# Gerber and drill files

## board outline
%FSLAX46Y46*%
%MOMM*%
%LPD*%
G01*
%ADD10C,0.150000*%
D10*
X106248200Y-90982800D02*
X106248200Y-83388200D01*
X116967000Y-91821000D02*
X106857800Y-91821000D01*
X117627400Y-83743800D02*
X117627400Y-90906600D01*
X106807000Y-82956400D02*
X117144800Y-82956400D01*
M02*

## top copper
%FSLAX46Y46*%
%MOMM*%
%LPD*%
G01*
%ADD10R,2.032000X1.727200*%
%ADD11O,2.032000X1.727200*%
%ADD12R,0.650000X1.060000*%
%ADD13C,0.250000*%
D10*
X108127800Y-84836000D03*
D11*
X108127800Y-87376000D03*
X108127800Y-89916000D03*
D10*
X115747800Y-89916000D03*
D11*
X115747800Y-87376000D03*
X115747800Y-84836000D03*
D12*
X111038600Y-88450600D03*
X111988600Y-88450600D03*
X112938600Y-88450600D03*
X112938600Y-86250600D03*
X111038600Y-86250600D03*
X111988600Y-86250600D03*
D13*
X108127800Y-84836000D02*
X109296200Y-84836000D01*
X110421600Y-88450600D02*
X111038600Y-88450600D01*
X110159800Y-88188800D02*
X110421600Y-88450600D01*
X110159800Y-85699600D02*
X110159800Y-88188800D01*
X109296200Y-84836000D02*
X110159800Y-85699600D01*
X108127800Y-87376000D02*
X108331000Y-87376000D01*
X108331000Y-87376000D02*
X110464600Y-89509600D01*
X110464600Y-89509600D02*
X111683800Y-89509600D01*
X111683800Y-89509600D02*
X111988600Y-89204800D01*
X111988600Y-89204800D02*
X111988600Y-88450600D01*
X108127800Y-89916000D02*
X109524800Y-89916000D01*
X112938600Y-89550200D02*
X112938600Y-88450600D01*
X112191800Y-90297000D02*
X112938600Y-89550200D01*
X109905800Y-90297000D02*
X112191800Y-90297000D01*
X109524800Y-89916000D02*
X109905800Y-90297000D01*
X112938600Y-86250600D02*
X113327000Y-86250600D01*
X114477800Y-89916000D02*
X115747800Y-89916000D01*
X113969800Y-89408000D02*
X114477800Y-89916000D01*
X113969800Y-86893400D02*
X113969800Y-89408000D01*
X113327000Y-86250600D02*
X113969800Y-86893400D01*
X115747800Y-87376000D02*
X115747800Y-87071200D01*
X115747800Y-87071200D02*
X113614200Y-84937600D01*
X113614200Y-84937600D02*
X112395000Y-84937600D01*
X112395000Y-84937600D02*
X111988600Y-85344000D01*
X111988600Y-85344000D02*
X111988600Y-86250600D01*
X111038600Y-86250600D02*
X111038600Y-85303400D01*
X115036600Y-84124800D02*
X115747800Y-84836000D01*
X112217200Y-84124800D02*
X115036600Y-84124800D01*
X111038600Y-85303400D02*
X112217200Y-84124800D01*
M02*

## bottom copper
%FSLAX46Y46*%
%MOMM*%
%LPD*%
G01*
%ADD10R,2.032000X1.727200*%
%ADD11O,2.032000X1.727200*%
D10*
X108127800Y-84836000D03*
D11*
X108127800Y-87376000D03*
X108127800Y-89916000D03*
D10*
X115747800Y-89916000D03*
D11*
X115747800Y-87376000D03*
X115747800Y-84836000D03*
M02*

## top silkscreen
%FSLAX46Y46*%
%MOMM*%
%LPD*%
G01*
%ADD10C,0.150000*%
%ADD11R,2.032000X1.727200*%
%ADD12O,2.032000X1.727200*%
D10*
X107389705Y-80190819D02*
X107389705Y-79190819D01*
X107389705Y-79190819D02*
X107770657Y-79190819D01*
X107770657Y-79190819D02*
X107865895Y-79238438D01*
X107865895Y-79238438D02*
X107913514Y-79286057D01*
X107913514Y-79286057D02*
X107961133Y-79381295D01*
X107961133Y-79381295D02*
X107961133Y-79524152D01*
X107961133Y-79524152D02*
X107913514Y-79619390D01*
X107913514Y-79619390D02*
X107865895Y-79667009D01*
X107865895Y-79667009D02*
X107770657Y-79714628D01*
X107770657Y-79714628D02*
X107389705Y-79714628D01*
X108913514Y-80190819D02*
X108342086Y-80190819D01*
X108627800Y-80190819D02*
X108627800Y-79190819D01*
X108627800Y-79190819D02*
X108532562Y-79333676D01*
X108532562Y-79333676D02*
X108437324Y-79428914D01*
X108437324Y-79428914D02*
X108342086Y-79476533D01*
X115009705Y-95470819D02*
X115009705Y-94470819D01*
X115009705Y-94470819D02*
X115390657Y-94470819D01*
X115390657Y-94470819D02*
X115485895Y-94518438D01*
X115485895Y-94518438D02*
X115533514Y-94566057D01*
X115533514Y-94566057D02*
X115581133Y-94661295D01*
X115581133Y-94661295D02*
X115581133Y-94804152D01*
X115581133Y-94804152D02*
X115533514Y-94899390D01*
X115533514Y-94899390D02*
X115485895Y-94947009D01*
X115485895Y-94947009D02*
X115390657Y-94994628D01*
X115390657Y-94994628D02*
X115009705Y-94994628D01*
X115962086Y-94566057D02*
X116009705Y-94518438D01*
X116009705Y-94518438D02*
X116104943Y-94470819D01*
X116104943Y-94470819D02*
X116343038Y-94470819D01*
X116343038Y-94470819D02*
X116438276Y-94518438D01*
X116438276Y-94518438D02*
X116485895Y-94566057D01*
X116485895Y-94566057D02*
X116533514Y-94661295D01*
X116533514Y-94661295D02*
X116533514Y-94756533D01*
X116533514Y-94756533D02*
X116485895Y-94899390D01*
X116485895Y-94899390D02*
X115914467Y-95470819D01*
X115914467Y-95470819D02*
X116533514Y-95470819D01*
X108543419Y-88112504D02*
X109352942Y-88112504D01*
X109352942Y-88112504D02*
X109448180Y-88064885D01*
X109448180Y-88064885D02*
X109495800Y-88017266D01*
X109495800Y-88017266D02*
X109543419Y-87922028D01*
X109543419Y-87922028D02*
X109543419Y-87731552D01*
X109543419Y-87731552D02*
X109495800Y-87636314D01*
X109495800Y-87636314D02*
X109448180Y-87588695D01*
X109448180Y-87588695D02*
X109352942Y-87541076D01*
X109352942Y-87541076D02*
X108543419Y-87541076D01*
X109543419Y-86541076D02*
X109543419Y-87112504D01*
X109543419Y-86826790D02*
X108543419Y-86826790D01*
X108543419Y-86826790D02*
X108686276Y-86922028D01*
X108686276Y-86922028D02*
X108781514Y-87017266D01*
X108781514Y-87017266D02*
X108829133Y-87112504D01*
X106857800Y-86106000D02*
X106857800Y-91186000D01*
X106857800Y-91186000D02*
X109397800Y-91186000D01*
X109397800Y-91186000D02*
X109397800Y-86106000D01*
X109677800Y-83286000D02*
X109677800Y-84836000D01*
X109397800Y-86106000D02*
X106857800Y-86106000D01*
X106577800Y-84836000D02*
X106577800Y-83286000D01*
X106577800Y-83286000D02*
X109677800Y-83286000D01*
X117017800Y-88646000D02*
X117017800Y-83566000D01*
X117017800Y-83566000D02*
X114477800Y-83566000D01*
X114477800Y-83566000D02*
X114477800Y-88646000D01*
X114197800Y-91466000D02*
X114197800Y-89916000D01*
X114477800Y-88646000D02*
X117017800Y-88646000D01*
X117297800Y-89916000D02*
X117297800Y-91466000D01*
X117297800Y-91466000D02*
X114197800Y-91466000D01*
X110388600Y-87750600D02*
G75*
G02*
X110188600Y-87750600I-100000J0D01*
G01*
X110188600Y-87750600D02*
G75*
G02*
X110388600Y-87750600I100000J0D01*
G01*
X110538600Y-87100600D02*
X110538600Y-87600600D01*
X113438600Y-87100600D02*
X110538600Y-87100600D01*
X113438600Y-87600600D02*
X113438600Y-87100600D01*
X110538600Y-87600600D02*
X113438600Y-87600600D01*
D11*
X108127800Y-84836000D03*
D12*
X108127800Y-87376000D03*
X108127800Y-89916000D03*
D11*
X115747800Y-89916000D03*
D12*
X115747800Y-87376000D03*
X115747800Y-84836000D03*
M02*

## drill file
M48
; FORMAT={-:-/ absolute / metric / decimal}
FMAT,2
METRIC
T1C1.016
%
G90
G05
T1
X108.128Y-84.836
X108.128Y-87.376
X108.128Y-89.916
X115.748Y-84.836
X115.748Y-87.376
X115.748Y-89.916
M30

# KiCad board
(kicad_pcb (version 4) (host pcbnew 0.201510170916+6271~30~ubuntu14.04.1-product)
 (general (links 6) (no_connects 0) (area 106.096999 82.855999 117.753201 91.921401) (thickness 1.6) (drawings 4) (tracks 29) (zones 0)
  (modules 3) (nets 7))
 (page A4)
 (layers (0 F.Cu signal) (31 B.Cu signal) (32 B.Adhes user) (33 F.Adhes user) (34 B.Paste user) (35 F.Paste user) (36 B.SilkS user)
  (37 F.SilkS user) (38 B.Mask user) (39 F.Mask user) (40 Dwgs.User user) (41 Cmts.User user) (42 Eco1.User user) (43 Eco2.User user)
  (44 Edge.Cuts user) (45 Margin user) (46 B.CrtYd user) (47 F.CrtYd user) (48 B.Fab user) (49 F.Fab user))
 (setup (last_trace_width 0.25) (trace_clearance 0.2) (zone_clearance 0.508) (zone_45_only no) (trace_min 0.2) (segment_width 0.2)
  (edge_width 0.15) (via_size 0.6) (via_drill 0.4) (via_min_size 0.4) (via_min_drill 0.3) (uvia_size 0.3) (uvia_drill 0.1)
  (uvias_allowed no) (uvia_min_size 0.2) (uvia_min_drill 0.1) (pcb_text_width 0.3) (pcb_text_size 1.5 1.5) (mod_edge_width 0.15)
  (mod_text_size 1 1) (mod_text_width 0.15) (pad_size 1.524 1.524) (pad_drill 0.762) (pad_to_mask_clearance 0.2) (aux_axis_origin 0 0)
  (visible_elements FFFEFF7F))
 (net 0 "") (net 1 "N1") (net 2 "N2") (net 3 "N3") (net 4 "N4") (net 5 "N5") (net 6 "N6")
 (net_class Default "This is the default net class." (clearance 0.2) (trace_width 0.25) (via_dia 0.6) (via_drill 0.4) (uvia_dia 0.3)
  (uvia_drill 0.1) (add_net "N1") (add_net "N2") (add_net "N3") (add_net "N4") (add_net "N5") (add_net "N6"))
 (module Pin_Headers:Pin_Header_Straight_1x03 (layer F.Cu) (at 108.1278 84.836)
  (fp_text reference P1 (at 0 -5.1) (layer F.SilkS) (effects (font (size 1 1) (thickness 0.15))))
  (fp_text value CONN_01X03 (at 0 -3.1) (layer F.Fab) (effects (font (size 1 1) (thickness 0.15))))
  (fp_line (start -1.27 1.27) (end -1.27 6.35) (layer F.SilkS) (width 0.15))
  (fp_line (start -1.27 6.35) (end 1.27 6.35) (layer F.SilkS) (width 0.15))
  (fp_line (start 1.27 6.35) (end 1.27 1.27) (layer F.SilkS) (width 0.15))
  (fp_line (start 1.55 -1.55) (end 1.55 0) (layer F.SilkS) (width 0.15))
  (fp_line (start 1.27 1.27) (end -1.27 1.27) (layer F.SilkS) (width 0.15))
  (fp_line (start -1.55 0) (end -1.55 -1.55) (layer F.SilkS) (width 0.15))
  (fp_line (start -1.55 -1.55) (end 1.55 -1.55) (layer F.SilkS) (width 0.15))
  (pad 1 thru_hole rect (at 0 0) (size 2.032 1.7272) (drill 1.016) (layers *.Cu *.Mask F.SilkS) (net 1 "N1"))
  (pad 2 thru_hole oval (at 0 2.54) (size 2.032 1.7272) (drill 1.016) (layers *.Cu *.Mask F.SilkS) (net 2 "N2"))
  (pad 3 thru_hole oval (at 0 5.08) (size 2.032 1.7272) (drill 1.016) (layers *.Cu *.Mask F.SilkS) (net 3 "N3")))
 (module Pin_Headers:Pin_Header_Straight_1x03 (layer F.Cu) (at 115.7478 89.916 180)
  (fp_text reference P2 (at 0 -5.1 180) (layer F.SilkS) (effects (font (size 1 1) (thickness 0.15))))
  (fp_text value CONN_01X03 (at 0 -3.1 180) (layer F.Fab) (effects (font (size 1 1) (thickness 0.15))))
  (fp_line (start -1.27 1.27) (end -1.27 6.35) (layer F.SilkS) (width 0.15))
  (fp_line (start -1.27 6.35) (end 1.27 6.35) (layer F.SilkS) (width 0.15))
  (fp_line (start 1.27 6.35) (end 1.27 1.27) (layer F.SilkS) (width 0.15))
  (fp_line (start 1.55 -1.55) (end 1.55 0) (layer F.SilkS) (width 0.15))
  (fp_line (start 1.27 1.27) (end -1.27 1.27) (layer F.SilkS) (width 0.15))
  (fp_line (start -1.55 0) (end -1.55 -1.55) (layer F.SilkS) (width 0.15))
  (fp_line (start -1.55 -1.55) (end 1.55 -1.55) (layer F.SilkS) (width 0.15))
  (pad 1 thru_hole rect (at 0 0 180) (size 2.032 1.7272) (drill 1.016) (layers *.Cu *.Mask F.SilkS) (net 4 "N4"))
  (pad 2 thru_hole oval (at 0 2.54 180) (size 2.032 1.7272) (drill 1.016) (layers *.Cu *.Mask F.SilkS) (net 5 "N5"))
  (pad 3 thru_hole oval (at 0 5.08 180) (size 2.032 1.7272) (drill 1.016) (layers *.Cu *.Mask F.SilkS) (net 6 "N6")))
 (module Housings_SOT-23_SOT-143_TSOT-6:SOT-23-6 (layer F.Cu) (at 111.9886 87.3506 90)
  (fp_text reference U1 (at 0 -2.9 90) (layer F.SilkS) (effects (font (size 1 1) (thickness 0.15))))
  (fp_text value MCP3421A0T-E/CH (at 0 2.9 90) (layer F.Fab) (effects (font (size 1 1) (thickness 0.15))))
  (fp_circle (center -0.4 -1.7) (end -0.3 -1.7) (layer F.SilkS) (width 0.15))
  (fp_line (start 0.25 -1.45) (end -0.25 -1.45) (layer F.SilkS) (width 0.15))
  (fp_line (start 0.25 1.45) (end 0.25 -1.45) (layer F.SilkS) (width 0.15))
  (fp_line (start -0.25 1.45) (end 0.25 1.45) (layer F.SilkS) (width 0.15))
  (fp_line (start -0.25 -1.45) (end -0.25 1.45) (layer F.SilkS) (width 0.15))
  (pad 1 smd rect (at -1.1 -0.95 90) (size 1.06 0.65) (layers F.Cu F.Paste F.Mask) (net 1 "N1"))
  (pad 2 smd rect (at -1.1 0 90) (size 1.06 0.65) (layers F.Cu F.Paste F.Mask) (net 2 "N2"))
  (pad 3 smd rect (at -1.1 0.95 90) (size 1.06 0.65) (layers F.Cu F.Paste F.Mask) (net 3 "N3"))
  (pad 4 smd rect (at 1.1 0.95 90) (size 1.06 0.65) (layers F.Cu F.Paste F.Mask) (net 4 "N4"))
  (pad 6 smd rect (at 1.1 -0.95 90) (size 1.06 0.65) (layers F.Cu F.Paste F.Mask) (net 6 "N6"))
  (pad 5 smd rect (at 1.1 0 90) (size 1.06 0.65) (layers F.Cu F.Paste F.Mask) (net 5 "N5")))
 (gr_line (start 106.2482 90.9828) (end 106.2482 83.3882) (angle 90) (layer Edge.Cuts) (width 0.15))
 (gr_line (start 116.967 91.821) (end 106.8578 91.821) (angle 90) (layer Edge.Cuts) (width 0.15))
 (gr_line (start 117.6274 83.7438) (end 117.6274 90.9066) (angle 90) (layer Edge.Cuts) (width 0.15))
 (gr_line (start 106.807 82.9564) (end 117.1448 82.9564) (angle 90) (layer Edge.Cuts) (width 0.15))
 (segment (start 108.1278 84.836) (end 109.2962 84.836) (width 0.25) (layer F.Cu) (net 1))
 (segment (start 110.4216 88.4506) (end 111.0386 88.4506) (width 0.25) (layer F.Cu) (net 1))
 (segment (start 110.1598 88.1888) (end 110.4216 88.4506) (width 0.25) (layer F.Cu) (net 1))
 (segment (start 110.1598 85.6996) (end 110.1598 88.1888) (width 0.25) (layer F.Cu) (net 1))
 (segment (start 109.2962 84.836) (end 110.1598 85.6996) (width 0.25) (layer F.Cu) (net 1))
 (segment (start 108.1278 87.376) (end 108.331 87.376) (width 0.25) (layer F.Cu) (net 2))
 (segment (start 108.331 87.376) (end 110.4646 89.5096) (width 0.25) (layer F.Cu) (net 2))
 (segment (start 110.4646 89.5096) (end 111.6838 89.5096) (width 0.25) (layer F.Cu) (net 2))
 (segment (start 111.6838 89.5096) (end 111.9886 89.2048) (width 0.25) (layer F.Cu) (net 2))
 (segment (start 111.9886 89.2048) (end 111.9886 88.4506) (width 0.25) (layer F.Cu) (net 2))
 (segment (start 108.1278 89.916) (end 109.5248 89.916) (width 0.25) (layer F.Cu) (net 3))
 (segment (start 112.9386 89.5502) (end 112.9386 88.4506) (width 0.25) (layer F.Cu) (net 3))
 (segment (start 112.1918 90.297) (end 112.9386 89.5502) (width 0.25) (layer F.Cu) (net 3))
 (segment (start 109.9058 90.297) (end 112.1918 90.297) (width 0.25) (layer F.Cu) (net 3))
 (segment (start 109.5248 89.916) (end 109.9058 90.297) (width 0.25) (layer F.Cu) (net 3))
 (segment (start 112.9386 86.2506) (end 113.327 86.2506) (width 0.25) (layer F.Cu) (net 4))
 (segment (start 114.4778 89.916) (end 115.7478 89.916) (width 0.25) (layer F.Cu) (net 4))
 (segment (start 113.9698 89.408) (end 114.4778 89.916) (width 0.25) (layer F.Cu) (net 4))
 (segment (start 113.9698 86.8934) (end 113.9698 89.408) (width 0.25) (layer F.Cu) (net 4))
 (segment (start 113.327 86.2506) (end 113.9698 86.8934) (width 0.25) (layer F.Cu) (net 4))
 (segment (start 115.7478 87.376) (end 115.7478 87.0712) (width 0.25) (layer F.Cu) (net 5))
 (segment (start 115.7478 87.0712) (end 113.6142 84.9376) (width 0.25) (layer F.Cu) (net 5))
 (segment (start 113.6142 84.9376) (end 112.395 84.9376) (width 0.25) (layer F.Cu) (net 5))
 (segment (start 112.395 84.9376) (end 111.9886 85.344) (width 0.25) (layer F.Cu) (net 5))
 (segment (start 111.9886 85.344) (end 111.9886 86.2506) (width 0.25) (layer F.Cu) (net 5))
 (segment (start 111.0386 86.2506) (end 111.0386 85.3034) (width 0.25) (layer F.Cu) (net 6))
 (segment (start 115.0366 84.1248) (end 115.7478 84.836) (width 0.25) (layer F.Cu) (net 6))
 (segment (start 112.2172 84.1248) (end 115.0366 84.1248) (width 0.25) (layer F.Cu) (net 6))
 (segment (start 111.0386 85.3034) (end 112.2172 84.1248) (width 0.25) (layer F.Cu) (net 6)))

